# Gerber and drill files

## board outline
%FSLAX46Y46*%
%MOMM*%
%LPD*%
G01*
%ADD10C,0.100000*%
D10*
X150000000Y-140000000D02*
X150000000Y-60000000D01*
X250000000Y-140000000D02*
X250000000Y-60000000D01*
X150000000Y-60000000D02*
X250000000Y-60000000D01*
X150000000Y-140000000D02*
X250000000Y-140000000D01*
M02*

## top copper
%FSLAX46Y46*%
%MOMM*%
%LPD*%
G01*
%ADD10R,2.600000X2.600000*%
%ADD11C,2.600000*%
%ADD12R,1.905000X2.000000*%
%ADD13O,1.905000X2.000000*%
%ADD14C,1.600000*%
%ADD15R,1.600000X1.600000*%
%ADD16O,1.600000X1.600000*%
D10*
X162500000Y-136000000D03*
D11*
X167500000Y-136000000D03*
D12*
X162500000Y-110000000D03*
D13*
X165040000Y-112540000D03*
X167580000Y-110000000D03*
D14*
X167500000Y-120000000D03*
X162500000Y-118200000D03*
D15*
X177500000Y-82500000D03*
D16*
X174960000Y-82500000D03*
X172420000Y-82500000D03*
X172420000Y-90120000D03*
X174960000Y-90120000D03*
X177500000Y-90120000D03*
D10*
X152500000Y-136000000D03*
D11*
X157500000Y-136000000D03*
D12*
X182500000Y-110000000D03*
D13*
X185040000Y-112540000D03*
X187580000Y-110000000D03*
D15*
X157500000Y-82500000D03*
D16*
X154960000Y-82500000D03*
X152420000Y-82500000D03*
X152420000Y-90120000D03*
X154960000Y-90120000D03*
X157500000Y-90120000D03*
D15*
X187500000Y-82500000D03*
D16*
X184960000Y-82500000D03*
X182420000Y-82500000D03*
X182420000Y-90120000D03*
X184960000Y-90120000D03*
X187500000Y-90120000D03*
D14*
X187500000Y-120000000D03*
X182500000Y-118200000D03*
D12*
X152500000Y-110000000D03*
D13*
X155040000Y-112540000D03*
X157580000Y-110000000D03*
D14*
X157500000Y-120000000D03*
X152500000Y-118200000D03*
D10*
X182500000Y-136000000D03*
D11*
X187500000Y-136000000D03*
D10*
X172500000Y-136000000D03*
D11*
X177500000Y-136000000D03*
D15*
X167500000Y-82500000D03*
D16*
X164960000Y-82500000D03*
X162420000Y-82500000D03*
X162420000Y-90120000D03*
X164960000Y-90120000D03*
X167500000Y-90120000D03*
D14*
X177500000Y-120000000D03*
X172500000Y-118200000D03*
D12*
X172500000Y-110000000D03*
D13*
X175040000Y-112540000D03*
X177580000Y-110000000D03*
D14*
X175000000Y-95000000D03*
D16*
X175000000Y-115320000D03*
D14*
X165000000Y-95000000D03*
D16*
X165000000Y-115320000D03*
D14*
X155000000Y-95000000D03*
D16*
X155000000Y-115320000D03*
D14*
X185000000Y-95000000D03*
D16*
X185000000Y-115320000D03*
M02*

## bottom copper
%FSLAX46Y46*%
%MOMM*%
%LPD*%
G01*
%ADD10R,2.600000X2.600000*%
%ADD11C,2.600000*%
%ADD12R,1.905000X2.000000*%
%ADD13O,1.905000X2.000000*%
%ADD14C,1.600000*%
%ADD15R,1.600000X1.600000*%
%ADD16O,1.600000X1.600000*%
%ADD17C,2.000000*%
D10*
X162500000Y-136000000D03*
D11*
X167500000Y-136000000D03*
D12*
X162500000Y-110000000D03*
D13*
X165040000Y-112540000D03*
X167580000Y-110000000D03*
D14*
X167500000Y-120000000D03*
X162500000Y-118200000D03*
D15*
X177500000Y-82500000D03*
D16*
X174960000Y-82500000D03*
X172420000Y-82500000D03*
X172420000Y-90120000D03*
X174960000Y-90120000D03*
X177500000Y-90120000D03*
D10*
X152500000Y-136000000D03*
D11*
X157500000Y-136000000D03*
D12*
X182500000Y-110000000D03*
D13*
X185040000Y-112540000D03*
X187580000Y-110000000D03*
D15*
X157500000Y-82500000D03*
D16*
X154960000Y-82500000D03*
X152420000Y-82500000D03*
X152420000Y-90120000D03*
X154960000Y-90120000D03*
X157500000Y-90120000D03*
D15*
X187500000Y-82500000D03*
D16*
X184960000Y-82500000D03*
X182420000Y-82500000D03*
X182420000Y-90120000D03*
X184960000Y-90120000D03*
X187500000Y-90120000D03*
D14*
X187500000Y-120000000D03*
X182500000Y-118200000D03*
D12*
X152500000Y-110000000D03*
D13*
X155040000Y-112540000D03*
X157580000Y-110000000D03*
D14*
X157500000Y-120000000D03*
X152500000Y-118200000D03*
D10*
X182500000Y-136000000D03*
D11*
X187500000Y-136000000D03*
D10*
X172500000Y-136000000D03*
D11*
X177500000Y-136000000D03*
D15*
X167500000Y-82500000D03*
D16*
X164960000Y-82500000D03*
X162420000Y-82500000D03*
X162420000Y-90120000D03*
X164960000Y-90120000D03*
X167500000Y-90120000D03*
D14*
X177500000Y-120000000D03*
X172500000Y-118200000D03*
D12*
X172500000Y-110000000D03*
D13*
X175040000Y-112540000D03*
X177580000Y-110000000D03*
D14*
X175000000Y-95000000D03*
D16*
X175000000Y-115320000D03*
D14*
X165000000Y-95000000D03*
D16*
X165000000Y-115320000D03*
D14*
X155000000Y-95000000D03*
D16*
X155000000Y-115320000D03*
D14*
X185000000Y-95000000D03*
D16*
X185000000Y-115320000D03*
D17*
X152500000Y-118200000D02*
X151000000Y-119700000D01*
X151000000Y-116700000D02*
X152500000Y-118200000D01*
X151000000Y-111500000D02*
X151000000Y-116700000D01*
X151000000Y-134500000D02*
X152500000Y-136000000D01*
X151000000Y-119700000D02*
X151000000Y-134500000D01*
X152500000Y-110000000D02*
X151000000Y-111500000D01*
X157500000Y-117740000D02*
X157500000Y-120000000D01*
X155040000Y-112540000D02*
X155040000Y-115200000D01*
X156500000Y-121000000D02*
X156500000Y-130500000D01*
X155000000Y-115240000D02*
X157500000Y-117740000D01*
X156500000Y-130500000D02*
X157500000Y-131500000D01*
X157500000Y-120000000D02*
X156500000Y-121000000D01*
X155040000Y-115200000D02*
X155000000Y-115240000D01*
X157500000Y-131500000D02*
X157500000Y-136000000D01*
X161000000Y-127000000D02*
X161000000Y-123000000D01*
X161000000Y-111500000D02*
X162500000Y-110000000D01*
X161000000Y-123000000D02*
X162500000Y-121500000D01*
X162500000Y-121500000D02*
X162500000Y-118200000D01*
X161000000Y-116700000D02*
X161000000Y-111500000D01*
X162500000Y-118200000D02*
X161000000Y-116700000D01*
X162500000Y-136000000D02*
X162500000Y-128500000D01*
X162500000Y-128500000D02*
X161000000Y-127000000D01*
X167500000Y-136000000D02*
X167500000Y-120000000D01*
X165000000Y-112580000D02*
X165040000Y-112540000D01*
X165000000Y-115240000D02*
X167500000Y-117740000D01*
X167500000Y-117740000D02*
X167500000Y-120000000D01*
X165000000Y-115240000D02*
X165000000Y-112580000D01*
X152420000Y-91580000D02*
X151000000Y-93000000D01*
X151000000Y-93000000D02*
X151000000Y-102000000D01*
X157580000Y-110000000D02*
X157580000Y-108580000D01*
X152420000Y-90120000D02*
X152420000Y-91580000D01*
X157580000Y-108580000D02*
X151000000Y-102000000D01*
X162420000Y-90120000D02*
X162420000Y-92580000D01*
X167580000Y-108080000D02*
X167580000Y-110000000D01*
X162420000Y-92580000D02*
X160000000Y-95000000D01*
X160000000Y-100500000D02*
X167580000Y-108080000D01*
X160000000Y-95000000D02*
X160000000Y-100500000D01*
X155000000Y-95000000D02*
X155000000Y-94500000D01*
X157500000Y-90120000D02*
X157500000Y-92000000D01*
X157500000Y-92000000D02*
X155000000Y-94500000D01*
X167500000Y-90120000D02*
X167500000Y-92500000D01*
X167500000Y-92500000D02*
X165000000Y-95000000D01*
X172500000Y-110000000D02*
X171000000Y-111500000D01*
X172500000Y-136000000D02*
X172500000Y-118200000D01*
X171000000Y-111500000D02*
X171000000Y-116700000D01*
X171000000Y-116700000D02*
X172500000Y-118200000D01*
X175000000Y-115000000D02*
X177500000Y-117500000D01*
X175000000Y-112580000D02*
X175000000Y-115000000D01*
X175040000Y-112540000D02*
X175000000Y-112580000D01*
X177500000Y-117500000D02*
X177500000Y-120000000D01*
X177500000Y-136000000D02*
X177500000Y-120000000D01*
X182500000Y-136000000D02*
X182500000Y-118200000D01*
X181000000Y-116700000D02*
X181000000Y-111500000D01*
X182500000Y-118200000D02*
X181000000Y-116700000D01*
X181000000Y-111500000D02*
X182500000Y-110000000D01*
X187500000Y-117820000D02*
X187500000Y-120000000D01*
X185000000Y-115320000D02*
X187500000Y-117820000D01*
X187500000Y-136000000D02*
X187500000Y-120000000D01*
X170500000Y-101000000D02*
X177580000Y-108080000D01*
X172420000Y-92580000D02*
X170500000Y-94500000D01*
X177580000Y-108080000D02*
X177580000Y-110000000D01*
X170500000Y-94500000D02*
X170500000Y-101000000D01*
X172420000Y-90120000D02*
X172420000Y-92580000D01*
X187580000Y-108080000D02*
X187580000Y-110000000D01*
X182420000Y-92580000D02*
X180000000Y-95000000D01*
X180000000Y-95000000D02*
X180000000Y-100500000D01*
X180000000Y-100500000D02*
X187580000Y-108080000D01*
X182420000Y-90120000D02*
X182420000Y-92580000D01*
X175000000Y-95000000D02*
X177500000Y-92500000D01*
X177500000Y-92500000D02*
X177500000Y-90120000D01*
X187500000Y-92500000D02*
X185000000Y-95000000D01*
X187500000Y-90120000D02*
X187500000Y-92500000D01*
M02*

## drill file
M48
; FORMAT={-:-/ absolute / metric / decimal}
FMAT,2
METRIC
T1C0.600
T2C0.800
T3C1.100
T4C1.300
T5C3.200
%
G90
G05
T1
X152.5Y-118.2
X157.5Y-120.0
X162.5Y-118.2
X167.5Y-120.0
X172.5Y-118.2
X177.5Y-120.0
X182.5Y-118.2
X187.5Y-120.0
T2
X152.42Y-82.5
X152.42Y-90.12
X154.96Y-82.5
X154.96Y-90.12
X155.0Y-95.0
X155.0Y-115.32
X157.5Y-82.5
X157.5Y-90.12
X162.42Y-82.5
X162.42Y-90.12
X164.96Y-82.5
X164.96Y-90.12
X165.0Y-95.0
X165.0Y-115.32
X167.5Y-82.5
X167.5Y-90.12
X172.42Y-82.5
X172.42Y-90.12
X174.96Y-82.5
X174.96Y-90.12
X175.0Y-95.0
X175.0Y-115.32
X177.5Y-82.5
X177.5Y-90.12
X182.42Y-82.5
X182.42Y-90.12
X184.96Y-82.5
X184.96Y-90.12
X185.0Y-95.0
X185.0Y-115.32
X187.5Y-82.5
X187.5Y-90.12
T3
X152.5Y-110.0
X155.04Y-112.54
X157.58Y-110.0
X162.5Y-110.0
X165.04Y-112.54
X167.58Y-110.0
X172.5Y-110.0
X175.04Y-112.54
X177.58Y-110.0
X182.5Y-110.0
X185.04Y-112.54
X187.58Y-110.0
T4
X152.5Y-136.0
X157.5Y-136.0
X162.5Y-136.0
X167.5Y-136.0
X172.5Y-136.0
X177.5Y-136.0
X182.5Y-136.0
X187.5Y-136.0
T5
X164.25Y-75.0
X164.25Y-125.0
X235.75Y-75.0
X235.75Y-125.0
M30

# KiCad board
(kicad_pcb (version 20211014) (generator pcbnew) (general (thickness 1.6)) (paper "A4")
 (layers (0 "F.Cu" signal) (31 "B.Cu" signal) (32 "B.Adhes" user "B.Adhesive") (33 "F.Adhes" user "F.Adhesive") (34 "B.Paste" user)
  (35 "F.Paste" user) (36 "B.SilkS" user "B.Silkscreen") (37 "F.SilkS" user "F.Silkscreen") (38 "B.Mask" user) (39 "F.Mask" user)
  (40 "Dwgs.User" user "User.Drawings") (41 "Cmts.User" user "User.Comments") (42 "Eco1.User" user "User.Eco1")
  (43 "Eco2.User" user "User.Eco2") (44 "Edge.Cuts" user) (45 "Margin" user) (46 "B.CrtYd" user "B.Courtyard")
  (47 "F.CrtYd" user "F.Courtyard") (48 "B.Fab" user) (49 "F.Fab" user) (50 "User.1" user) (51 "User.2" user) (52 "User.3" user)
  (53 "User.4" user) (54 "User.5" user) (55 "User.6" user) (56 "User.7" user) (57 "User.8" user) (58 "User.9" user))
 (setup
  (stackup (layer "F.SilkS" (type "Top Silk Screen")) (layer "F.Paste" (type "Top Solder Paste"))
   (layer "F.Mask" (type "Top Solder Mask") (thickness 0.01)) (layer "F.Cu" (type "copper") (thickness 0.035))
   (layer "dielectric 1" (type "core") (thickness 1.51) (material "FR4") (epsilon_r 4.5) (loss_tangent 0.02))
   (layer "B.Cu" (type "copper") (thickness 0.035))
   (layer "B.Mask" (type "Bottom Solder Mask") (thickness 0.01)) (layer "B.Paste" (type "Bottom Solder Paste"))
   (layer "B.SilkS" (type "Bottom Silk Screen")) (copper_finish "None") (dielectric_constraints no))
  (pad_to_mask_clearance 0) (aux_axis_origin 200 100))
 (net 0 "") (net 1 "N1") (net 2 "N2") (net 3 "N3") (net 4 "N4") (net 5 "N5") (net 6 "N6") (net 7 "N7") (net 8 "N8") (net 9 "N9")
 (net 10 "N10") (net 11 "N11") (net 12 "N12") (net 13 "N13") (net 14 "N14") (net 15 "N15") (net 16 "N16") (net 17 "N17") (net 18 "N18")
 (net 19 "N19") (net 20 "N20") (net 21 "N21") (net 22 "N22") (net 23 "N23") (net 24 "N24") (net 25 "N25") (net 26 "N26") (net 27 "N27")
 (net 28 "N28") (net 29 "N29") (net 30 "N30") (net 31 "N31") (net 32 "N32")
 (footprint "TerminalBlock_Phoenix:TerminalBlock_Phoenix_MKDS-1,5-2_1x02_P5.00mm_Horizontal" (layer "F.Cu") (at 162.5 136)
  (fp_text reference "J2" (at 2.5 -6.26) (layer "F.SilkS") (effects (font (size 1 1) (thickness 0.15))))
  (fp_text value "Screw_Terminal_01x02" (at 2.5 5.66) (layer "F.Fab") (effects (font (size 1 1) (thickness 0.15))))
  (pad "1" thru_hole rect (at 0 0) (size 2.6 2.6) (drill 1.3) (layers *.Cu *.Mask) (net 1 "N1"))
  (pad "2" thru_hole circle (at 5 0) (size 2.6 2.6) (drill 1.3) (layers *.Cu *.Mask) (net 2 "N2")))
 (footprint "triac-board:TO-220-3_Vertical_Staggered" (layer "F.Cu") (at 162.5 110)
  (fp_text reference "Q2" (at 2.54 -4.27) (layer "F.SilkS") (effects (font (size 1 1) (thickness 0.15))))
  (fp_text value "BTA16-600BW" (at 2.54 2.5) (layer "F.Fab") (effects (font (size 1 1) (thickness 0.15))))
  (pad "1" thru_hole rect (at 0 0) (size 1.905 2) (drill 1.1) (layers *.Cu *.Mask) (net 1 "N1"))
  (pad "2" thru_hole oval (at 2.54 2.54) (size 1.905 2) (drill 1.1) (layers *.Cu *.Mask) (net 2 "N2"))
  (pad "3" thru_hole oval (at 5.08 0) (size 1.905 2) (drill 1.1) (layers *.Cu *.Mask) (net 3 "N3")))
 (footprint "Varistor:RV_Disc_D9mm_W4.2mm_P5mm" (layer "F.Cu") (at 167.5 120 180)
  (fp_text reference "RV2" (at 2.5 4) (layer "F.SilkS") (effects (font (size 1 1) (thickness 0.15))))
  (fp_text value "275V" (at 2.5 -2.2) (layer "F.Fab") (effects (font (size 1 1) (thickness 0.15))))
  (pad "1" thru_hole circle (at 0 0 180) (size 1.6 1.6) (drill 0.6) (layers *.Cu *.Mask) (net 2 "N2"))
  (pad "2" thru_hole circle (at 5 1.8 180) (size 1.6 1.6) (drill 0.6) (layers *.Cu *.Mask) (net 1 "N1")))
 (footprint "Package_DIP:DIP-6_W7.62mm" (layer "F.Cu") (at 177.5 82.5 -90)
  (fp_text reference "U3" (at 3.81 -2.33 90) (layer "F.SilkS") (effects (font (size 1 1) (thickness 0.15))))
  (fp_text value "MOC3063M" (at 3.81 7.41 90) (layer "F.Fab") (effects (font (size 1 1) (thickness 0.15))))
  (pad "1" thru_hole rect (at 0 0 270) (size 1.6 1.6) (drill 0.8) (layers *.Cu *.Mask) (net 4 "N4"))
  (pad "2" thru_hole oval (at 0 2.54 270) (size 1.6 1.6) (drill 0.8) (layers *.Cu *.Mask) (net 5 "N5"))
  (pad "3" thru_hole oval (at 0 5.08 270) (size 1.6 1.6) (drill 0.8) (layers *.Cu *.Mask) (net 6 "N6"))
  (pad "4" thru_hole oval (at 7.62 5.08 270) (size 1.6 1.6) (drill 0.8) (layers *.Cu *.Mask) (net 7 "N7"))
  (pad "5" thru_hole oval (at 7.62 2.54 270) (size 1.6 1.6) (drill 0.8) (layers *.Cu *.Mask) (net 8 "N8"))
  (pad "6" thru_hole oval (at 7.62 0 270) (size 1.6 1.6) (drill 0.8) (layers *.Cu *.Mask) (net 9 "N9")))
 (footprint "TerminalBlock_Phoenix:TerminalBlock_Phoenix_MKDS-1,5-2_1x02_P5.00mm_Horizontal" (layer "F.Cu") (at 152.5 136)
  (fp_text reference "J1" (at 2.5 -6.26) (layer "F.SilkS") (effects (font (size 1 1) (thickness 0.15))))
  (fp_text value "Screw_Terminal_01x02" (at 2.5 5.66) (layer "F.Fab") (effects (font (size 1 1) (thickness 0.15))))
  (pad "1" thru_hole rect (at 0 0) (size 2.6 2.6) (drill 1.3) (layers *.Cu *.Mask) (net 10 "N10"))
  (pad "2" thru_hole circle (at 5 0) (size 2.6 2.6) (drill 1.3) (layers *.Cu *.Mask) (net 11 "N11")))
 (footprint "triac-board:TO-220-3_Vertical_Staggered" (layer "F.Cu") (at 182.5 110)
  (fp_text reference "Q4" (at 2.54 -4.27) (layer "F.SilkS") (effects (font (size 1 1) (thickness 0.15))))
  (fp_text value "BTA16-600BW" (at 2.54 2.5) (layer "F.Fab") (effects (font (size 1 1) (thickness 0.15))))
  (pad "1" thru_hole rect (at 0 0) (size 1.905 2) (drill 1.1) (layers *.Cu *.Mask) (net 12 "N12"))
  (pad "2" thru_hole oval (at 2.54 2.54) (size 1.905 2) (drill 1.1) (layers *.Cu *.Mask) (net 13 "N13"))
  (pad "3" thru_hole oval (at 5.08 0) (size 1.905 2) (drill 1.1) (layers *.Cu *.Mask) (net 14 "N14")))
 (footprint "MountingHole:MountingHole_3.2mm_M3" (layer "F.Cu") (at 235.75 75)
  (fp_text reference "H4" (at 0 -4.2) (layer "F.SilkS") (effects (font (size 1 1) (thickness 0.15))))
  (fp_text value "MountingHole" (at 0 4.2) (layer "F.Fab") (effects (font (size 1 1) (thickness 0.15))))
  (pad "" np_thru_hole circle (at 0 0) (size 3.2 3.2) (drill 3.2) (layers *.Cu *.Mask)))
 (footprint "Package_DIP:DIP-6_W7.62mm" (layer "F.Cu") (at 157.5 82.5 -90)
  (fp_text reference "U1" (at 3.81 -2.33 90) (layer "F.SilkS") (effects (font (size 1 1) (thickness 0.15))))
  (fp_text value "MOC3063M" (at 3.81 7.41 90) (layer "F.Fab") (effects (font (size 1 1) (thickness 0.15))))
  (pad "1" thru_hole rect (at 0 0 270) (size 1.6 1.6) (drill 0.8) (layers *.Cu *.Mask) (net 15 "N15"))
  (pad "2" thru_hole oval (at 0 2.54 270) (size 1.6 1.6) (drill 0.8) (layers *.Cu *.Mask) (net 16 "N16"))
  (pad "3" thru_hole oval (at 0 5.08 270) (size 1.6 1.6) (drill 0.8) (layers *.Cu *.Mask) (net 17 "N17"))
  (pad "4" thru_hole oval (at 7.62 5.08 270) (size 1.6 1.6) (drill 0.8) (layers *.Cu *.Mask) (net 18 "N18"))
  (pad "5" thru_hole oval (at 7.62 2.54 270) (size 1.6 1.6) (drill 0.8) (layers *.Cu *.Mask) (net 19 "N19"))
  (pad "6" thru_hole oval (at 7.62 0 270) (size 1.6 1.6) (drill 0.8) (layers *.Cu *.Mask) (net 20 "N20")))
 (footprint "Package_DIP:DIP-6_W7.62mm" (layer "F.Cu") (at 187.5 82.5 -90)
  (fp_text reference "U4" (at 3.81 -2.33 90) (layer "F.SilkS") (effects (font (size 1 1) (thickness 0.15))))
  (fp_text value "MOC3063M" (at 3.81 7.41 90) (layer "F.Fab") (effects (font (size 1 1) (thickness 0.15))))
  (pad "1" thru_hole rect (at 0 0 270) (size 1.6 1.6) (drill 0.8) (layers *.Cu *.Mask) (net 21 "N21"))
  (pad "2" thru_hole oval (at 0 2.54 270) (size 1.6 1.6) (drill 0.8) (layers *.Cu *.Mask) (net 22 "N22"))
  (pad "3" thru_hole oval (at 0 5.08 270) (size 1.6 1.6) (drill 0.8) (layers *.Cu *.Mask) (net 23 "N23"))
  (pad "4" thru_hole oval (at 7.62 5.08 270) (size 1.6 1.6) (drill 0.8) (layers *.Cu *.Mask) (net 14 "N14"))
  (pad "5" thru_hole oval (at 7.62 2.54 270) (size 1.6 1.6) (drill 0.8) (layers *.Cu *.Mask) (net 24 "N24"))
  (pad "6" thru_hole oval (at 7.62 0 270) (size 1.6 1.6) (drill 0.8) (layers *.Cu *.Mask) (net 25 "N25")))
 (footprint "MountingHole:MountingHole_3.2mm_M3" (layer "F.Cu") (at 235.75 125)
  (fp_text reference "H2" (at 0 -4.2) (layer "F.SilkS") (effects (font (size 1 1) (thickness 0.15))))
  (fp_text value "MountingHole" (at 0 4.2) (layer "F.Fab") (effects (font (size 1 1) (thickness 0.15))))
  (pad "" np_thru_hole circle (at 0 0) (size 3.2 3.2) (drill 3.2) (layers *.Cu *.Mask)))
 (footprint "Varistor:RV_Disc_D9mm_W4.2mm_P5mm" (layer "F.Cu") (at 187.5 120 180)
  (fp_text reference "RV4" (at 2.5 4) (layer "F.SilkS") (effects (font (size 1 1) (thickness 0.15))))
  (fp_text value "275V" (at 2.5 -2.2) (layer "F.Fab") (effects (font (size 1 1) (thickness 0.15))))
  (pad "1" thru_hole circle (at 0 0 180) (size 1.6 1.6) (drill 0.6) (layers *.Cu *.Mask) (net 13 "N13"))
  (pad "2" thru_hole circle (at 5 1.8 180) (size 1.6 1.6) (drill 0.6) (layers *.Cu *.Mask) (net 12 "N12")))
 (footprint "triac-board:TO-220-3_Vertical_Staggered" (layer "F.Cu") (at 152.5 110)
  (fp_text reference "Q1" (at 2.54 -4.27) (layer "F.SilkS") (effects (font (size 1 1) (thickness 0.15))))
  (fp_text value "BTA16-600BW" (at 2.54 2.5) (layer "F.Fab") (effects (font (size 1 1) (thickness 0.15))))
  (pad "1" thru_hole rect (at 0 0) (size 1.905 2) (drill 1.1) (layers *.Cu *.Mask) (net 10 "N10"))
  (pad "2" thru_hole oval (at 2.54 2.54) (size 1.905 2) (drill 1.1) (layers *.Cu *.Mask) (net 11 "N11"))
  (pad "3" thru_hole oval (at 5.08 0) (size 1.905 2) (drill 1.1) (layers *.Cu *.Mask) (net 18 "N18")))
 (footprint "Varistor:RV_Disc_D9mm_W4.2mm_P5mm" (layer "F.Cu") (at 157.5 120 180)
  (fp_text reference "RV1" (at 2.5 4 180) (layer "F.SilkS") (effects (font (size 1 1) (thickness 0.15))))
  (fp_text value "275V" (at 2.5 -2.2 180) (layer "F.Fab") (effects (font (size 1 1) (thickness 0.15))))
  (pad "1" thru_hole circle (at 0 0 180) (size 1.6 1.6) (drill 0.6) (layers *.Cu *.Mask) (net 11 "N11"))
  (pad "2" thru_hole circle (at 5 1.8 180) (size 1.6 1.6) (drill 0.6) (layers *.Cu *.Mask) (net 10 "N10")))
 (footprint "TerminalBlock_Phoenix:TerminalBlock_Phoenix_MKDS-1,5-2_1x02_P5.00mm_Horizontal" (layer "F.Cu") (at 182.5 136)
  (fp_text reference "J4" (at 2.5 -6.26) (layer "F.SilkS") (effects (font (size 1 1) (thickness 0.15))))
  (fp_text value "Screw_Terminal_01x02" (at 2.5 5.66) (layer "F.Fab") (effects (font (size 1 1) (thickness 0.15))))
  (pad "1" thru_hole rect (at 0 0) (size 2.6 2.6) (drill 1.3) (layers *.Cu *.Mask) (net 12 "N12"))
  (pad "2" thru_hole circle (at 5 0) (size 2.6 2.6) (drill 1.3) (layers *.Cu *.Mask) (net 13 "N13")))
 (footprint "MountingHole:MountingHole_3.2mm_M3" (layer "F.Cu") (at 164.25 125)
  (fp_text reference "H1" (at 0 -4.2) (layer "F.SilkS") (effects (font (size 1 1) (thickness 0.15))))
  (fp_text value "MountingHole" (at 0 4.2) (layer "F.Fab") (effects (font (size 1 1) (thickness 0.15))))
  (pad "" np_thru_hole circle (at 0 0) (size 3.2 3.2) (drill 3.2) (layers *.Cu *.Mask)))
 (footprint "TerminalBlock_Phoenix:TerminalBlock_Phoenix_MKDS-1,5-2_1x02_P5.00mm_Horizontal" (layer "F.Cu") (at 172.5 136)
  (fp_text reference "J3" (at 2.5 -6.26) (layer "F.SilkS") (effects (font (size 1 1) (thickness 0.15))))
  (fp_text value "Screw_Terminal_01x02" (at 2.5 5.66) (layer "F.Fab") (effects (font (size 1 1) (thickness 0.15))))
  (pad "1" thru_hole rect (at 0 0) (size 2.6 2.6) (drill 1.3) (layers *.Cu *.Mask) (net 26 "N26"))
  (pad "2" thru_hole circle (at 5 0) (size 2.6 2.6) (drill 1.3) (layers *.Cu *.Mask) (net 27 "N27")))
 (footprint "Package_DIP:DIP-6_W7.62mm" (layer "F.Cu") (at 167.5 82.5 -90)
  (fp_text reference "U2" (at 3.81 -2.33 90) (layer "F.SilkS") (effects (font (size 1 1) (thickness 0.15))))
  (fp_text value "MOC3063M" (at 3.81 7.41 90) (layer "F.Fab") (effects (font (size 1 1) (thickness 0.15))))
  (pad "1" thru_hole rect (at 0 0 270) (size 1.6 1.6) (drill 0.8) (layers *.Cu *.Mask) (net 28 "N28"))
  (pad "2" thru_hole oval (at 0 2.54 270) (size 1.6 1.6) (drill 0.8) (layers *.Cu *.Mask) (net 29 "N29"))
  (pad "3" thru_hole oval (at 0 5.08 270) (size 1.6 1.6) (drill 0.8) (layers *.Cu *.Mask) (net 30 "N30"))
  (pad "4" thru_hole oval (at 7.62 5.08 270) (size 1.6 1.6) (drill 0.8) (layers *.Cu *.Mask) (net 3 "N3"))
  (pad "5" thru_hole oval (at 7.62 2.54 270) (size 1.6 1.6) (drill 0.8) (layers *.Cu *.Mask) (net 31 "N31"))
  (pad "6" thru_hole oval (at 7.62 0 270) (size 1.6 1.6) (drill 0.8) (layers *.Cu *.Mask) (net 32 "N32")))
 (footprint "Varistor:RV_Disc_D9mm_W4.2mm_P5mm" (layer "F.Cu") (at 177.5 120 180)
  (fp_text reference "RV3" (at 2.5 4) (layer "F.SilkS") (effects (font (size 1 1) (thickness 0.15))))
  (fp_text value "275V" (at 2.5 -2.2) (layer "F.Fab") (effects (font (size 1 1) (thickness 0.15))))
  (pad "1" thru_hole circle (at 0 0 180) (size 1.6 1.6) (drill 0.6) (layers *.Cu *.Mask) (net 27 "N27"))
  (pad "2" thru_hole circle (at 5 1.8 180) (size 1.6 1.6) (drill 0.6) (layers *.Cu *.Mask) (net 26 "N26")))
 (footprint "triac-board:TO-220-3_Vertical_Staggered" (layer "F.Cu") (at 172.5 110)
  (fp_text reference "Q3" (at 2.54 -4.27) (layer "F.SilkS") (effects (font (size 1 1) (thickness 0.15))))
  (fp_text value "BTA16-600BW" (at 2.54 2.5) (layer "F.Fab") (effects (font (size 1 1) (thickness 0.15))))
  (pad "1" thru_hole rect (at 0 0) (size 1.905 2) (drill 1.1) (layers *.Cu *.Mask) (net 26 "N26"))
  (pad "2" thru_hole oval (at 2.54 2.54) (size 1.905 2) (drill 1.1) (layers *.Cu *.Mask) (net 27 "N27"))
  (pad "3" thru_hole oval (at 5.08 0) (size 1.905 2) (drill 1.1) (layers *.Cu *.Mask) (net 7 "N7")))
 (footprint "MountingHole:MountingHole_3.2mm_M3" (layer "F.Cu") (at 164.25 75)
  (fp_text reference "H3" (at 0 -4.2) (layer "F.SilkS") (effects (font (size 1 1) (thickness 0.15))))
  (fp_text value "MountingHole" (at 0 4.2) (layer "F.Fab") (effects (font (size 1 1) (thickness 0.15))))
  (pad "" np_thru_hole circle (at 0 0) (size 3.2 3.2) (drill 3.2) (layers *.Cu *.Mask)))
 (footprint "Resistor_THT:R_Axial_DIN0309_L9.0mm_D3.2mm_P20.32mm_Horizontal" (layer "B.Cu") (at 175 95 -90)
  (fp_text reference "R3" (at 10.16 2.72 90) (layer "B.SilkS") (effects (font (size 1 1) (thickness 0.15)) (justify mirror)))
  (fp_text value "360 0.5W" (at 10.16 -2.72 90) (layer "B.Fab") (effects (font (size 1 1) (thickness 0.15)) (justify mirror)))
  (pad "1" thru_hole circle (at 0 0 270) (size 1.6 1.6) (drill 0.8) (layers *.Cu *.Mask) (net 9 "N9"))
  (pad "2" thru_hole oval (at 20.32 0 270) (size 1.6 1.6) (drill 0.8) (layers *.Cu *.Mask) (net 27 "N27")))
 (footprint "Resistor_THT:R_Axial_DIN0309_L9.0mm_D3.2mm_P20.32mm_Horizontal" (layer "B.Cu") (at 165 95 -90)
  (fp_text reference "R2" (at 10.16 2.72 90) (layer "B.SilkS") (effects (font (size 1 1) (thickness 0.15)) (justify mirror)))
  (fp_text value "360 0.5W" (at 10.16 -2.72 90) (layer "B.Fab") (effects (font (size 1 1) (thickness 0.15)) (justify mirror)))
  (pad "1" thru_hole circle (at 0 0 270) (size 1.6 1.6) (drill 0.8) (layers *.Cu *.Mask) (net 32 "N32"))
  (pad "2" thru_hole oval (at 20.32 0 270) (size 1.6 1.6) (drill 0.8) (layers *.Cu *.Mask) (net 2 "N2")))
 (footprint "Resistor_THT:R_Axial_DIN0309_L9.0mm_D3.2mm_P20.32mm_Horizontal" (layer "B.Cu") (at 155 95 -90)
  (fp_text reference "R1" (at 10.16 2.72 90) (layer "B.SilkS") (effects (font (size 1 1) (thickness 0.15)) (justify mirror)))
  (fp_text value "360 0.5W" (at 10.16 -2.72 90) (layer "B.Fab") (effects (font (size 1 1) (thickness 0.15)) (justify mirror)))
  (pad "1" thru_hole circle (at 0 0 270) (size 1.6 1.6) (drill 0.8) (layers *.Cu *.Mask) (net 20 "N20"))
  (pad "2" thru_hole oval (at 20.32 0 270) (size 1.6 1.6) (drill 0.8) (layers *.Cu *.Mask) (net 11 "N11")))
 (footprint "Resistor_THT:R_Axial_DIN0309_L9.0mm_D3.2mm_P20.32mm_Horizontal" (layer "B.Cu") (at 185 95 -90)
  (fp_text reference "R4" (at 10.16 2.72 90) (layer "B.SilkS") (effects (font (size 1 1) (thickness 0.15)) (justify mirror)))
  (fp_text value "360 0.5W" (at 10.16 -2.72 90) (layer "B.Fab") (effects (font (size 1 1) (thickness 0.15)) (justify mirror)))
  (pad "1" thru_hole circle (at 0 0 270) (size 1.6 1.6) (drill 0.8) (layers *.Cu *.Mask) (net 25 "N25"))
  (pad "2" thru_hole oval (at 20.32 0 270) (size 1.6 1.6) (drill 0.8) (layers *.Cu *.Mask) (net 13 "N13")))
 (gr_line (start 150 140) (end 150 60) (layer "Edge.Cuts") (width 0.1))
 (gr_line (start 250 140) (end 250 60) (layer "Edge.Cuts") (width 0.1))
 (gr_line (start 150 60) (end 250 60) (layer "Edge.Cuts") (width 0.1))
 (gr_line (start 150 140) (end 250 140) (layer "Edge.Cuts") (width 0.1))
 (segment (start 152.5 118.2) (end 151 119.7) (width 2) (layer "B.Cu") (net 10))
 (segment (start 151 116.7) (end 152.5 118.2) (width 2) (layer "B.Cu") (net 10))
 (segment (start 151 111.5) (end 151 116.7) (width 2) (layer "B.Cu") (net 10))
 (segment (start 151 134.5) (end 152.5 136) (width 2) (layer "B.Cu") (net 10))
 (segment (start 151 119.7) (end 151 134.5) (width 2) (layer "B.Cu") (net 10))
 (segment (start 152.5 110) (end 151 111.5) (width 2) (layer "B.Cu") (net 10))
 (segment (start 157.5 117.74) (end 157.5 120) (width 2) (layer "B.Cu") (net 11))
 (segment (start 155.04 112.54) (end 155.04 115.2) (width 2) (layer "B.Cu") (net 11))
 (segment (start 156.5 121) (end 156.5 130.5) (width 2) (layer "B.Cu") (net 11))
 (segment (start 155 115.24) (end 157.5 117.74) (width 2) (layer "B.Cu") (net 11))
 (segment (start 156.5 130.5) (end 157.5 131.5) (width 2) (layer "B.Cu") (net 11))
 (segment (start 157.5 120) (end 156.5 121) (width 2) (layer "B.Cu") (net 11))
 (segment (start 155.04 115.2) (end 155 115.24) (width 2) (layer "B.Cu") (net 11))
 (segment (start 157.5 131.5) (end 157.5 136) (width 2) (layer "B.Cu") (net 11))
 (segment (start 161 127) (end 161 123) (width 2) (layer "B.Cu") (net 1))
 (segment (start 161 111.5) (end 162.5 110) (width 2) (layer "B.Cu") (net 1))
 (segment (start 161 123) (end 162.5 121.5) (width 2) (layer "B.Cu") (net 1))
 (segment (start 162.5 121.5) (end 162.5 118.2) (width 2) (layer "B.Cu") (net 1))
 (segment (start 161 116.7) (end 161 111.5) (width 2) (layer "B.Cu") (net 1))
 (segment (start 162.5 118.2) (end 161 116.7) (width 2) (layer "B.Cu") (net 1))
 (segment (start 162.5 136) (end 162.5 128.5) (width 2) (layer "B.Cu") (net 1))
 (segment (start 162.5 128.5) (end 161 127) (width 2) (layer "B.Cu") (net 1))
 (segment (start 167.5 136) (end 167.5 120) (width 2) (layer "B.Cu") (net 2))
 (segment (start 165 112.58) (end 165.04 112.54) (width 2) (layer "B.Cu") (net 2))
 (segment (start 165 115.24) (end 167.5 117.74) (width 2) (layer "B.Cu") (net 2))
 (segment (start 167.5 117.74) (end 167.5 120) (width 2) (layer "B.Cu") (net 2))
 (segment (start 165 115.24) (end 165 112.58) (width 2) (layer "B.Cu") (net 2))
 (segment (start 152.42 91.58) (end 151 93) (width 2) (layer "B.Cu") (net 18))
 (segment (start 151 93) (end 151 102) (width 2) (layer "B.Cu") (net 18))
 (segment (start 157.58 110) (end 157.58 108.58) (width 2) (layer "B.Cu") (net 18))
 (segment (start 152.42 90.12) (end 152.42 91.58) (width 2) (layer "B.Cu") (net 18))
 (segment (start 157.58 108.58) (end 151 102) (width 2) (layer "B.Cu") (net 18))
 (segment (start 162.42 90.12) (end 162.42 92.58) (width 2) (layer "B.Cu") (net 3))
 (segment (start 167.58 108.08) (end 167.58 110) (width 2) (layer "B.Cu") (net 3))
 (segment (start 162.42 92.58) (end 160 95) (width 2) (layer "B.Cu") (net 3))
 (segment (start 160 100.5) (end 167.58 108.08) (width 2) (layer "B.Cu") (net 3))
 (segment (start 160 95) (end 160 100.5) (width 2) (layer "B.Cu") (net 3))
 (segment (start 155 95) (end 155 94.5) (width 2) (layer "B.Cu") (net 20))
 (segment (start 157.5 90.12) (end 157.5 92) (width 2) (layer "B.Cu") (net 20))
 (segment (start 157.5 92) (end 155 94.5) (width 2) (layer "B.Cu") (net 20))
 (segment (start 167.5 90.12) (end 167.5 92.5) (width 2) (layer "B.Cu") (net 32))
 (segment (start 167.5 92.5) (end 165 95) (width 2) (layer "B.Cu") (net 32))
 (segment (start 172.5 110) (end 171 111.5) (width 2) (layer "B.Cu") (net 26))
 (segment (start 172.5 136) (end 172.5 118.2) (width 2) (layer "B.Cu") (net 26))
 (segment (start 171 111.5) (end 171 116.7) (width 2) (layer "B.Cu") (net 26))
 (segment (start 171 116.7) (end 172.5 118.2) (width 2) (layer "B.Cu") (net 26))
 (segment (start 175 115) (end 177.5 117.5) (width 2) (layer "B.Cu") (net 27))
 (segment (start 175 112.58) (end 175 115) (width 2) (layer "B.Cu") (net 27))
 (segment (start 175.04 112.54) (end 175 112.58) (width 2) (layer "B.Cu") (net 27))
 (segment (start 177.5 117.5) (end 177.5 120) (width 2) (layer "B.Cu") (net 27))
 (segment (start 177.5 136) (end 177.5 120) (width 2) (layer "B.Cu") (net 27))
 (segment (start 182.5 136) (end 182.5 118.2) (width 2) (layer "B.Cu") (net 12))
 (segment (start 181 116.7) (end 181 111.5) (width 2) (layer "B.Cu") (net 12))
 (segment (start 182.5 118.2) (end 181 116.7) (width 2) (layer "B.Cu") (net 12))
 (segment (start 181 111.5) (end 182.5 110) (width 2) (layer "B.Cu") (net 12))
 (segment (start 187.5 117.82) (end 187.5 120) (width 2) (layer "B.Cu") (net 13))
 (segment (start 185 115.32) (end 187.5 117.82) (width 2) (layer "B.Cu") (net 13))
 (segment (start 187.5 136) (end 187.5 120) (width 2) (layer "B.Cu") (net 13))
 (segment (start 170.5 101) (end 177.58 108.08) (width 2) (layer "B.Cu") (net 7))
 (segment (start 172.42 92.58) (end 170.5 94.5) (width 2) (layer "B.Cu") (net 7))
 (segment (start 177.58 108.08) (end 177.58 110) (width 2) (layer "B.Cu") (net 7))
 (segment (start 170.5 94.5) (end 170.5 101) (width 2) (layer "B.Cu") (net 7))
 (segment (start 172.42 90.12) (end 172.42 92.58) (width 2) (layer "B.Cu") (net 7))
 (segment (start 187.58 108.08) (end 187.58 110) (width 2) (layer "B.Cu") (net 14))
 (segment (start 182.42 92.58) (end 180 95) (width 2) (layer "B.Cu") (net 14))
 (segment (start 180 95) (end 180 100.5) (width 2) (layer "B.Cu") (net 14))
 (segment (start 180 100.5) (end 187.58 108.08) (width 2) (layer "B.Cu") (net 14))
 (segment (start 182.42 90.12) (end 182.42 92.58) (width 2) (layer "B.Cu") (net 14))
 (segment (start 175 95) (end 177.5 92.5) (width 2) (layer "B.Cu") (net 9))
 (segment (start 177.5 92.5) (end 177.5 90.12) (width 2) (layer "B.Cu") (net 9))
 (segment (start 187.5 92.5) (end 185 95) (width 2) (layer "B.Cu") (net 25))
 (segment (start 187.5 90.12) (end 187.5 92.5) (width 2) (layer "B.Cu") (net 25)))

